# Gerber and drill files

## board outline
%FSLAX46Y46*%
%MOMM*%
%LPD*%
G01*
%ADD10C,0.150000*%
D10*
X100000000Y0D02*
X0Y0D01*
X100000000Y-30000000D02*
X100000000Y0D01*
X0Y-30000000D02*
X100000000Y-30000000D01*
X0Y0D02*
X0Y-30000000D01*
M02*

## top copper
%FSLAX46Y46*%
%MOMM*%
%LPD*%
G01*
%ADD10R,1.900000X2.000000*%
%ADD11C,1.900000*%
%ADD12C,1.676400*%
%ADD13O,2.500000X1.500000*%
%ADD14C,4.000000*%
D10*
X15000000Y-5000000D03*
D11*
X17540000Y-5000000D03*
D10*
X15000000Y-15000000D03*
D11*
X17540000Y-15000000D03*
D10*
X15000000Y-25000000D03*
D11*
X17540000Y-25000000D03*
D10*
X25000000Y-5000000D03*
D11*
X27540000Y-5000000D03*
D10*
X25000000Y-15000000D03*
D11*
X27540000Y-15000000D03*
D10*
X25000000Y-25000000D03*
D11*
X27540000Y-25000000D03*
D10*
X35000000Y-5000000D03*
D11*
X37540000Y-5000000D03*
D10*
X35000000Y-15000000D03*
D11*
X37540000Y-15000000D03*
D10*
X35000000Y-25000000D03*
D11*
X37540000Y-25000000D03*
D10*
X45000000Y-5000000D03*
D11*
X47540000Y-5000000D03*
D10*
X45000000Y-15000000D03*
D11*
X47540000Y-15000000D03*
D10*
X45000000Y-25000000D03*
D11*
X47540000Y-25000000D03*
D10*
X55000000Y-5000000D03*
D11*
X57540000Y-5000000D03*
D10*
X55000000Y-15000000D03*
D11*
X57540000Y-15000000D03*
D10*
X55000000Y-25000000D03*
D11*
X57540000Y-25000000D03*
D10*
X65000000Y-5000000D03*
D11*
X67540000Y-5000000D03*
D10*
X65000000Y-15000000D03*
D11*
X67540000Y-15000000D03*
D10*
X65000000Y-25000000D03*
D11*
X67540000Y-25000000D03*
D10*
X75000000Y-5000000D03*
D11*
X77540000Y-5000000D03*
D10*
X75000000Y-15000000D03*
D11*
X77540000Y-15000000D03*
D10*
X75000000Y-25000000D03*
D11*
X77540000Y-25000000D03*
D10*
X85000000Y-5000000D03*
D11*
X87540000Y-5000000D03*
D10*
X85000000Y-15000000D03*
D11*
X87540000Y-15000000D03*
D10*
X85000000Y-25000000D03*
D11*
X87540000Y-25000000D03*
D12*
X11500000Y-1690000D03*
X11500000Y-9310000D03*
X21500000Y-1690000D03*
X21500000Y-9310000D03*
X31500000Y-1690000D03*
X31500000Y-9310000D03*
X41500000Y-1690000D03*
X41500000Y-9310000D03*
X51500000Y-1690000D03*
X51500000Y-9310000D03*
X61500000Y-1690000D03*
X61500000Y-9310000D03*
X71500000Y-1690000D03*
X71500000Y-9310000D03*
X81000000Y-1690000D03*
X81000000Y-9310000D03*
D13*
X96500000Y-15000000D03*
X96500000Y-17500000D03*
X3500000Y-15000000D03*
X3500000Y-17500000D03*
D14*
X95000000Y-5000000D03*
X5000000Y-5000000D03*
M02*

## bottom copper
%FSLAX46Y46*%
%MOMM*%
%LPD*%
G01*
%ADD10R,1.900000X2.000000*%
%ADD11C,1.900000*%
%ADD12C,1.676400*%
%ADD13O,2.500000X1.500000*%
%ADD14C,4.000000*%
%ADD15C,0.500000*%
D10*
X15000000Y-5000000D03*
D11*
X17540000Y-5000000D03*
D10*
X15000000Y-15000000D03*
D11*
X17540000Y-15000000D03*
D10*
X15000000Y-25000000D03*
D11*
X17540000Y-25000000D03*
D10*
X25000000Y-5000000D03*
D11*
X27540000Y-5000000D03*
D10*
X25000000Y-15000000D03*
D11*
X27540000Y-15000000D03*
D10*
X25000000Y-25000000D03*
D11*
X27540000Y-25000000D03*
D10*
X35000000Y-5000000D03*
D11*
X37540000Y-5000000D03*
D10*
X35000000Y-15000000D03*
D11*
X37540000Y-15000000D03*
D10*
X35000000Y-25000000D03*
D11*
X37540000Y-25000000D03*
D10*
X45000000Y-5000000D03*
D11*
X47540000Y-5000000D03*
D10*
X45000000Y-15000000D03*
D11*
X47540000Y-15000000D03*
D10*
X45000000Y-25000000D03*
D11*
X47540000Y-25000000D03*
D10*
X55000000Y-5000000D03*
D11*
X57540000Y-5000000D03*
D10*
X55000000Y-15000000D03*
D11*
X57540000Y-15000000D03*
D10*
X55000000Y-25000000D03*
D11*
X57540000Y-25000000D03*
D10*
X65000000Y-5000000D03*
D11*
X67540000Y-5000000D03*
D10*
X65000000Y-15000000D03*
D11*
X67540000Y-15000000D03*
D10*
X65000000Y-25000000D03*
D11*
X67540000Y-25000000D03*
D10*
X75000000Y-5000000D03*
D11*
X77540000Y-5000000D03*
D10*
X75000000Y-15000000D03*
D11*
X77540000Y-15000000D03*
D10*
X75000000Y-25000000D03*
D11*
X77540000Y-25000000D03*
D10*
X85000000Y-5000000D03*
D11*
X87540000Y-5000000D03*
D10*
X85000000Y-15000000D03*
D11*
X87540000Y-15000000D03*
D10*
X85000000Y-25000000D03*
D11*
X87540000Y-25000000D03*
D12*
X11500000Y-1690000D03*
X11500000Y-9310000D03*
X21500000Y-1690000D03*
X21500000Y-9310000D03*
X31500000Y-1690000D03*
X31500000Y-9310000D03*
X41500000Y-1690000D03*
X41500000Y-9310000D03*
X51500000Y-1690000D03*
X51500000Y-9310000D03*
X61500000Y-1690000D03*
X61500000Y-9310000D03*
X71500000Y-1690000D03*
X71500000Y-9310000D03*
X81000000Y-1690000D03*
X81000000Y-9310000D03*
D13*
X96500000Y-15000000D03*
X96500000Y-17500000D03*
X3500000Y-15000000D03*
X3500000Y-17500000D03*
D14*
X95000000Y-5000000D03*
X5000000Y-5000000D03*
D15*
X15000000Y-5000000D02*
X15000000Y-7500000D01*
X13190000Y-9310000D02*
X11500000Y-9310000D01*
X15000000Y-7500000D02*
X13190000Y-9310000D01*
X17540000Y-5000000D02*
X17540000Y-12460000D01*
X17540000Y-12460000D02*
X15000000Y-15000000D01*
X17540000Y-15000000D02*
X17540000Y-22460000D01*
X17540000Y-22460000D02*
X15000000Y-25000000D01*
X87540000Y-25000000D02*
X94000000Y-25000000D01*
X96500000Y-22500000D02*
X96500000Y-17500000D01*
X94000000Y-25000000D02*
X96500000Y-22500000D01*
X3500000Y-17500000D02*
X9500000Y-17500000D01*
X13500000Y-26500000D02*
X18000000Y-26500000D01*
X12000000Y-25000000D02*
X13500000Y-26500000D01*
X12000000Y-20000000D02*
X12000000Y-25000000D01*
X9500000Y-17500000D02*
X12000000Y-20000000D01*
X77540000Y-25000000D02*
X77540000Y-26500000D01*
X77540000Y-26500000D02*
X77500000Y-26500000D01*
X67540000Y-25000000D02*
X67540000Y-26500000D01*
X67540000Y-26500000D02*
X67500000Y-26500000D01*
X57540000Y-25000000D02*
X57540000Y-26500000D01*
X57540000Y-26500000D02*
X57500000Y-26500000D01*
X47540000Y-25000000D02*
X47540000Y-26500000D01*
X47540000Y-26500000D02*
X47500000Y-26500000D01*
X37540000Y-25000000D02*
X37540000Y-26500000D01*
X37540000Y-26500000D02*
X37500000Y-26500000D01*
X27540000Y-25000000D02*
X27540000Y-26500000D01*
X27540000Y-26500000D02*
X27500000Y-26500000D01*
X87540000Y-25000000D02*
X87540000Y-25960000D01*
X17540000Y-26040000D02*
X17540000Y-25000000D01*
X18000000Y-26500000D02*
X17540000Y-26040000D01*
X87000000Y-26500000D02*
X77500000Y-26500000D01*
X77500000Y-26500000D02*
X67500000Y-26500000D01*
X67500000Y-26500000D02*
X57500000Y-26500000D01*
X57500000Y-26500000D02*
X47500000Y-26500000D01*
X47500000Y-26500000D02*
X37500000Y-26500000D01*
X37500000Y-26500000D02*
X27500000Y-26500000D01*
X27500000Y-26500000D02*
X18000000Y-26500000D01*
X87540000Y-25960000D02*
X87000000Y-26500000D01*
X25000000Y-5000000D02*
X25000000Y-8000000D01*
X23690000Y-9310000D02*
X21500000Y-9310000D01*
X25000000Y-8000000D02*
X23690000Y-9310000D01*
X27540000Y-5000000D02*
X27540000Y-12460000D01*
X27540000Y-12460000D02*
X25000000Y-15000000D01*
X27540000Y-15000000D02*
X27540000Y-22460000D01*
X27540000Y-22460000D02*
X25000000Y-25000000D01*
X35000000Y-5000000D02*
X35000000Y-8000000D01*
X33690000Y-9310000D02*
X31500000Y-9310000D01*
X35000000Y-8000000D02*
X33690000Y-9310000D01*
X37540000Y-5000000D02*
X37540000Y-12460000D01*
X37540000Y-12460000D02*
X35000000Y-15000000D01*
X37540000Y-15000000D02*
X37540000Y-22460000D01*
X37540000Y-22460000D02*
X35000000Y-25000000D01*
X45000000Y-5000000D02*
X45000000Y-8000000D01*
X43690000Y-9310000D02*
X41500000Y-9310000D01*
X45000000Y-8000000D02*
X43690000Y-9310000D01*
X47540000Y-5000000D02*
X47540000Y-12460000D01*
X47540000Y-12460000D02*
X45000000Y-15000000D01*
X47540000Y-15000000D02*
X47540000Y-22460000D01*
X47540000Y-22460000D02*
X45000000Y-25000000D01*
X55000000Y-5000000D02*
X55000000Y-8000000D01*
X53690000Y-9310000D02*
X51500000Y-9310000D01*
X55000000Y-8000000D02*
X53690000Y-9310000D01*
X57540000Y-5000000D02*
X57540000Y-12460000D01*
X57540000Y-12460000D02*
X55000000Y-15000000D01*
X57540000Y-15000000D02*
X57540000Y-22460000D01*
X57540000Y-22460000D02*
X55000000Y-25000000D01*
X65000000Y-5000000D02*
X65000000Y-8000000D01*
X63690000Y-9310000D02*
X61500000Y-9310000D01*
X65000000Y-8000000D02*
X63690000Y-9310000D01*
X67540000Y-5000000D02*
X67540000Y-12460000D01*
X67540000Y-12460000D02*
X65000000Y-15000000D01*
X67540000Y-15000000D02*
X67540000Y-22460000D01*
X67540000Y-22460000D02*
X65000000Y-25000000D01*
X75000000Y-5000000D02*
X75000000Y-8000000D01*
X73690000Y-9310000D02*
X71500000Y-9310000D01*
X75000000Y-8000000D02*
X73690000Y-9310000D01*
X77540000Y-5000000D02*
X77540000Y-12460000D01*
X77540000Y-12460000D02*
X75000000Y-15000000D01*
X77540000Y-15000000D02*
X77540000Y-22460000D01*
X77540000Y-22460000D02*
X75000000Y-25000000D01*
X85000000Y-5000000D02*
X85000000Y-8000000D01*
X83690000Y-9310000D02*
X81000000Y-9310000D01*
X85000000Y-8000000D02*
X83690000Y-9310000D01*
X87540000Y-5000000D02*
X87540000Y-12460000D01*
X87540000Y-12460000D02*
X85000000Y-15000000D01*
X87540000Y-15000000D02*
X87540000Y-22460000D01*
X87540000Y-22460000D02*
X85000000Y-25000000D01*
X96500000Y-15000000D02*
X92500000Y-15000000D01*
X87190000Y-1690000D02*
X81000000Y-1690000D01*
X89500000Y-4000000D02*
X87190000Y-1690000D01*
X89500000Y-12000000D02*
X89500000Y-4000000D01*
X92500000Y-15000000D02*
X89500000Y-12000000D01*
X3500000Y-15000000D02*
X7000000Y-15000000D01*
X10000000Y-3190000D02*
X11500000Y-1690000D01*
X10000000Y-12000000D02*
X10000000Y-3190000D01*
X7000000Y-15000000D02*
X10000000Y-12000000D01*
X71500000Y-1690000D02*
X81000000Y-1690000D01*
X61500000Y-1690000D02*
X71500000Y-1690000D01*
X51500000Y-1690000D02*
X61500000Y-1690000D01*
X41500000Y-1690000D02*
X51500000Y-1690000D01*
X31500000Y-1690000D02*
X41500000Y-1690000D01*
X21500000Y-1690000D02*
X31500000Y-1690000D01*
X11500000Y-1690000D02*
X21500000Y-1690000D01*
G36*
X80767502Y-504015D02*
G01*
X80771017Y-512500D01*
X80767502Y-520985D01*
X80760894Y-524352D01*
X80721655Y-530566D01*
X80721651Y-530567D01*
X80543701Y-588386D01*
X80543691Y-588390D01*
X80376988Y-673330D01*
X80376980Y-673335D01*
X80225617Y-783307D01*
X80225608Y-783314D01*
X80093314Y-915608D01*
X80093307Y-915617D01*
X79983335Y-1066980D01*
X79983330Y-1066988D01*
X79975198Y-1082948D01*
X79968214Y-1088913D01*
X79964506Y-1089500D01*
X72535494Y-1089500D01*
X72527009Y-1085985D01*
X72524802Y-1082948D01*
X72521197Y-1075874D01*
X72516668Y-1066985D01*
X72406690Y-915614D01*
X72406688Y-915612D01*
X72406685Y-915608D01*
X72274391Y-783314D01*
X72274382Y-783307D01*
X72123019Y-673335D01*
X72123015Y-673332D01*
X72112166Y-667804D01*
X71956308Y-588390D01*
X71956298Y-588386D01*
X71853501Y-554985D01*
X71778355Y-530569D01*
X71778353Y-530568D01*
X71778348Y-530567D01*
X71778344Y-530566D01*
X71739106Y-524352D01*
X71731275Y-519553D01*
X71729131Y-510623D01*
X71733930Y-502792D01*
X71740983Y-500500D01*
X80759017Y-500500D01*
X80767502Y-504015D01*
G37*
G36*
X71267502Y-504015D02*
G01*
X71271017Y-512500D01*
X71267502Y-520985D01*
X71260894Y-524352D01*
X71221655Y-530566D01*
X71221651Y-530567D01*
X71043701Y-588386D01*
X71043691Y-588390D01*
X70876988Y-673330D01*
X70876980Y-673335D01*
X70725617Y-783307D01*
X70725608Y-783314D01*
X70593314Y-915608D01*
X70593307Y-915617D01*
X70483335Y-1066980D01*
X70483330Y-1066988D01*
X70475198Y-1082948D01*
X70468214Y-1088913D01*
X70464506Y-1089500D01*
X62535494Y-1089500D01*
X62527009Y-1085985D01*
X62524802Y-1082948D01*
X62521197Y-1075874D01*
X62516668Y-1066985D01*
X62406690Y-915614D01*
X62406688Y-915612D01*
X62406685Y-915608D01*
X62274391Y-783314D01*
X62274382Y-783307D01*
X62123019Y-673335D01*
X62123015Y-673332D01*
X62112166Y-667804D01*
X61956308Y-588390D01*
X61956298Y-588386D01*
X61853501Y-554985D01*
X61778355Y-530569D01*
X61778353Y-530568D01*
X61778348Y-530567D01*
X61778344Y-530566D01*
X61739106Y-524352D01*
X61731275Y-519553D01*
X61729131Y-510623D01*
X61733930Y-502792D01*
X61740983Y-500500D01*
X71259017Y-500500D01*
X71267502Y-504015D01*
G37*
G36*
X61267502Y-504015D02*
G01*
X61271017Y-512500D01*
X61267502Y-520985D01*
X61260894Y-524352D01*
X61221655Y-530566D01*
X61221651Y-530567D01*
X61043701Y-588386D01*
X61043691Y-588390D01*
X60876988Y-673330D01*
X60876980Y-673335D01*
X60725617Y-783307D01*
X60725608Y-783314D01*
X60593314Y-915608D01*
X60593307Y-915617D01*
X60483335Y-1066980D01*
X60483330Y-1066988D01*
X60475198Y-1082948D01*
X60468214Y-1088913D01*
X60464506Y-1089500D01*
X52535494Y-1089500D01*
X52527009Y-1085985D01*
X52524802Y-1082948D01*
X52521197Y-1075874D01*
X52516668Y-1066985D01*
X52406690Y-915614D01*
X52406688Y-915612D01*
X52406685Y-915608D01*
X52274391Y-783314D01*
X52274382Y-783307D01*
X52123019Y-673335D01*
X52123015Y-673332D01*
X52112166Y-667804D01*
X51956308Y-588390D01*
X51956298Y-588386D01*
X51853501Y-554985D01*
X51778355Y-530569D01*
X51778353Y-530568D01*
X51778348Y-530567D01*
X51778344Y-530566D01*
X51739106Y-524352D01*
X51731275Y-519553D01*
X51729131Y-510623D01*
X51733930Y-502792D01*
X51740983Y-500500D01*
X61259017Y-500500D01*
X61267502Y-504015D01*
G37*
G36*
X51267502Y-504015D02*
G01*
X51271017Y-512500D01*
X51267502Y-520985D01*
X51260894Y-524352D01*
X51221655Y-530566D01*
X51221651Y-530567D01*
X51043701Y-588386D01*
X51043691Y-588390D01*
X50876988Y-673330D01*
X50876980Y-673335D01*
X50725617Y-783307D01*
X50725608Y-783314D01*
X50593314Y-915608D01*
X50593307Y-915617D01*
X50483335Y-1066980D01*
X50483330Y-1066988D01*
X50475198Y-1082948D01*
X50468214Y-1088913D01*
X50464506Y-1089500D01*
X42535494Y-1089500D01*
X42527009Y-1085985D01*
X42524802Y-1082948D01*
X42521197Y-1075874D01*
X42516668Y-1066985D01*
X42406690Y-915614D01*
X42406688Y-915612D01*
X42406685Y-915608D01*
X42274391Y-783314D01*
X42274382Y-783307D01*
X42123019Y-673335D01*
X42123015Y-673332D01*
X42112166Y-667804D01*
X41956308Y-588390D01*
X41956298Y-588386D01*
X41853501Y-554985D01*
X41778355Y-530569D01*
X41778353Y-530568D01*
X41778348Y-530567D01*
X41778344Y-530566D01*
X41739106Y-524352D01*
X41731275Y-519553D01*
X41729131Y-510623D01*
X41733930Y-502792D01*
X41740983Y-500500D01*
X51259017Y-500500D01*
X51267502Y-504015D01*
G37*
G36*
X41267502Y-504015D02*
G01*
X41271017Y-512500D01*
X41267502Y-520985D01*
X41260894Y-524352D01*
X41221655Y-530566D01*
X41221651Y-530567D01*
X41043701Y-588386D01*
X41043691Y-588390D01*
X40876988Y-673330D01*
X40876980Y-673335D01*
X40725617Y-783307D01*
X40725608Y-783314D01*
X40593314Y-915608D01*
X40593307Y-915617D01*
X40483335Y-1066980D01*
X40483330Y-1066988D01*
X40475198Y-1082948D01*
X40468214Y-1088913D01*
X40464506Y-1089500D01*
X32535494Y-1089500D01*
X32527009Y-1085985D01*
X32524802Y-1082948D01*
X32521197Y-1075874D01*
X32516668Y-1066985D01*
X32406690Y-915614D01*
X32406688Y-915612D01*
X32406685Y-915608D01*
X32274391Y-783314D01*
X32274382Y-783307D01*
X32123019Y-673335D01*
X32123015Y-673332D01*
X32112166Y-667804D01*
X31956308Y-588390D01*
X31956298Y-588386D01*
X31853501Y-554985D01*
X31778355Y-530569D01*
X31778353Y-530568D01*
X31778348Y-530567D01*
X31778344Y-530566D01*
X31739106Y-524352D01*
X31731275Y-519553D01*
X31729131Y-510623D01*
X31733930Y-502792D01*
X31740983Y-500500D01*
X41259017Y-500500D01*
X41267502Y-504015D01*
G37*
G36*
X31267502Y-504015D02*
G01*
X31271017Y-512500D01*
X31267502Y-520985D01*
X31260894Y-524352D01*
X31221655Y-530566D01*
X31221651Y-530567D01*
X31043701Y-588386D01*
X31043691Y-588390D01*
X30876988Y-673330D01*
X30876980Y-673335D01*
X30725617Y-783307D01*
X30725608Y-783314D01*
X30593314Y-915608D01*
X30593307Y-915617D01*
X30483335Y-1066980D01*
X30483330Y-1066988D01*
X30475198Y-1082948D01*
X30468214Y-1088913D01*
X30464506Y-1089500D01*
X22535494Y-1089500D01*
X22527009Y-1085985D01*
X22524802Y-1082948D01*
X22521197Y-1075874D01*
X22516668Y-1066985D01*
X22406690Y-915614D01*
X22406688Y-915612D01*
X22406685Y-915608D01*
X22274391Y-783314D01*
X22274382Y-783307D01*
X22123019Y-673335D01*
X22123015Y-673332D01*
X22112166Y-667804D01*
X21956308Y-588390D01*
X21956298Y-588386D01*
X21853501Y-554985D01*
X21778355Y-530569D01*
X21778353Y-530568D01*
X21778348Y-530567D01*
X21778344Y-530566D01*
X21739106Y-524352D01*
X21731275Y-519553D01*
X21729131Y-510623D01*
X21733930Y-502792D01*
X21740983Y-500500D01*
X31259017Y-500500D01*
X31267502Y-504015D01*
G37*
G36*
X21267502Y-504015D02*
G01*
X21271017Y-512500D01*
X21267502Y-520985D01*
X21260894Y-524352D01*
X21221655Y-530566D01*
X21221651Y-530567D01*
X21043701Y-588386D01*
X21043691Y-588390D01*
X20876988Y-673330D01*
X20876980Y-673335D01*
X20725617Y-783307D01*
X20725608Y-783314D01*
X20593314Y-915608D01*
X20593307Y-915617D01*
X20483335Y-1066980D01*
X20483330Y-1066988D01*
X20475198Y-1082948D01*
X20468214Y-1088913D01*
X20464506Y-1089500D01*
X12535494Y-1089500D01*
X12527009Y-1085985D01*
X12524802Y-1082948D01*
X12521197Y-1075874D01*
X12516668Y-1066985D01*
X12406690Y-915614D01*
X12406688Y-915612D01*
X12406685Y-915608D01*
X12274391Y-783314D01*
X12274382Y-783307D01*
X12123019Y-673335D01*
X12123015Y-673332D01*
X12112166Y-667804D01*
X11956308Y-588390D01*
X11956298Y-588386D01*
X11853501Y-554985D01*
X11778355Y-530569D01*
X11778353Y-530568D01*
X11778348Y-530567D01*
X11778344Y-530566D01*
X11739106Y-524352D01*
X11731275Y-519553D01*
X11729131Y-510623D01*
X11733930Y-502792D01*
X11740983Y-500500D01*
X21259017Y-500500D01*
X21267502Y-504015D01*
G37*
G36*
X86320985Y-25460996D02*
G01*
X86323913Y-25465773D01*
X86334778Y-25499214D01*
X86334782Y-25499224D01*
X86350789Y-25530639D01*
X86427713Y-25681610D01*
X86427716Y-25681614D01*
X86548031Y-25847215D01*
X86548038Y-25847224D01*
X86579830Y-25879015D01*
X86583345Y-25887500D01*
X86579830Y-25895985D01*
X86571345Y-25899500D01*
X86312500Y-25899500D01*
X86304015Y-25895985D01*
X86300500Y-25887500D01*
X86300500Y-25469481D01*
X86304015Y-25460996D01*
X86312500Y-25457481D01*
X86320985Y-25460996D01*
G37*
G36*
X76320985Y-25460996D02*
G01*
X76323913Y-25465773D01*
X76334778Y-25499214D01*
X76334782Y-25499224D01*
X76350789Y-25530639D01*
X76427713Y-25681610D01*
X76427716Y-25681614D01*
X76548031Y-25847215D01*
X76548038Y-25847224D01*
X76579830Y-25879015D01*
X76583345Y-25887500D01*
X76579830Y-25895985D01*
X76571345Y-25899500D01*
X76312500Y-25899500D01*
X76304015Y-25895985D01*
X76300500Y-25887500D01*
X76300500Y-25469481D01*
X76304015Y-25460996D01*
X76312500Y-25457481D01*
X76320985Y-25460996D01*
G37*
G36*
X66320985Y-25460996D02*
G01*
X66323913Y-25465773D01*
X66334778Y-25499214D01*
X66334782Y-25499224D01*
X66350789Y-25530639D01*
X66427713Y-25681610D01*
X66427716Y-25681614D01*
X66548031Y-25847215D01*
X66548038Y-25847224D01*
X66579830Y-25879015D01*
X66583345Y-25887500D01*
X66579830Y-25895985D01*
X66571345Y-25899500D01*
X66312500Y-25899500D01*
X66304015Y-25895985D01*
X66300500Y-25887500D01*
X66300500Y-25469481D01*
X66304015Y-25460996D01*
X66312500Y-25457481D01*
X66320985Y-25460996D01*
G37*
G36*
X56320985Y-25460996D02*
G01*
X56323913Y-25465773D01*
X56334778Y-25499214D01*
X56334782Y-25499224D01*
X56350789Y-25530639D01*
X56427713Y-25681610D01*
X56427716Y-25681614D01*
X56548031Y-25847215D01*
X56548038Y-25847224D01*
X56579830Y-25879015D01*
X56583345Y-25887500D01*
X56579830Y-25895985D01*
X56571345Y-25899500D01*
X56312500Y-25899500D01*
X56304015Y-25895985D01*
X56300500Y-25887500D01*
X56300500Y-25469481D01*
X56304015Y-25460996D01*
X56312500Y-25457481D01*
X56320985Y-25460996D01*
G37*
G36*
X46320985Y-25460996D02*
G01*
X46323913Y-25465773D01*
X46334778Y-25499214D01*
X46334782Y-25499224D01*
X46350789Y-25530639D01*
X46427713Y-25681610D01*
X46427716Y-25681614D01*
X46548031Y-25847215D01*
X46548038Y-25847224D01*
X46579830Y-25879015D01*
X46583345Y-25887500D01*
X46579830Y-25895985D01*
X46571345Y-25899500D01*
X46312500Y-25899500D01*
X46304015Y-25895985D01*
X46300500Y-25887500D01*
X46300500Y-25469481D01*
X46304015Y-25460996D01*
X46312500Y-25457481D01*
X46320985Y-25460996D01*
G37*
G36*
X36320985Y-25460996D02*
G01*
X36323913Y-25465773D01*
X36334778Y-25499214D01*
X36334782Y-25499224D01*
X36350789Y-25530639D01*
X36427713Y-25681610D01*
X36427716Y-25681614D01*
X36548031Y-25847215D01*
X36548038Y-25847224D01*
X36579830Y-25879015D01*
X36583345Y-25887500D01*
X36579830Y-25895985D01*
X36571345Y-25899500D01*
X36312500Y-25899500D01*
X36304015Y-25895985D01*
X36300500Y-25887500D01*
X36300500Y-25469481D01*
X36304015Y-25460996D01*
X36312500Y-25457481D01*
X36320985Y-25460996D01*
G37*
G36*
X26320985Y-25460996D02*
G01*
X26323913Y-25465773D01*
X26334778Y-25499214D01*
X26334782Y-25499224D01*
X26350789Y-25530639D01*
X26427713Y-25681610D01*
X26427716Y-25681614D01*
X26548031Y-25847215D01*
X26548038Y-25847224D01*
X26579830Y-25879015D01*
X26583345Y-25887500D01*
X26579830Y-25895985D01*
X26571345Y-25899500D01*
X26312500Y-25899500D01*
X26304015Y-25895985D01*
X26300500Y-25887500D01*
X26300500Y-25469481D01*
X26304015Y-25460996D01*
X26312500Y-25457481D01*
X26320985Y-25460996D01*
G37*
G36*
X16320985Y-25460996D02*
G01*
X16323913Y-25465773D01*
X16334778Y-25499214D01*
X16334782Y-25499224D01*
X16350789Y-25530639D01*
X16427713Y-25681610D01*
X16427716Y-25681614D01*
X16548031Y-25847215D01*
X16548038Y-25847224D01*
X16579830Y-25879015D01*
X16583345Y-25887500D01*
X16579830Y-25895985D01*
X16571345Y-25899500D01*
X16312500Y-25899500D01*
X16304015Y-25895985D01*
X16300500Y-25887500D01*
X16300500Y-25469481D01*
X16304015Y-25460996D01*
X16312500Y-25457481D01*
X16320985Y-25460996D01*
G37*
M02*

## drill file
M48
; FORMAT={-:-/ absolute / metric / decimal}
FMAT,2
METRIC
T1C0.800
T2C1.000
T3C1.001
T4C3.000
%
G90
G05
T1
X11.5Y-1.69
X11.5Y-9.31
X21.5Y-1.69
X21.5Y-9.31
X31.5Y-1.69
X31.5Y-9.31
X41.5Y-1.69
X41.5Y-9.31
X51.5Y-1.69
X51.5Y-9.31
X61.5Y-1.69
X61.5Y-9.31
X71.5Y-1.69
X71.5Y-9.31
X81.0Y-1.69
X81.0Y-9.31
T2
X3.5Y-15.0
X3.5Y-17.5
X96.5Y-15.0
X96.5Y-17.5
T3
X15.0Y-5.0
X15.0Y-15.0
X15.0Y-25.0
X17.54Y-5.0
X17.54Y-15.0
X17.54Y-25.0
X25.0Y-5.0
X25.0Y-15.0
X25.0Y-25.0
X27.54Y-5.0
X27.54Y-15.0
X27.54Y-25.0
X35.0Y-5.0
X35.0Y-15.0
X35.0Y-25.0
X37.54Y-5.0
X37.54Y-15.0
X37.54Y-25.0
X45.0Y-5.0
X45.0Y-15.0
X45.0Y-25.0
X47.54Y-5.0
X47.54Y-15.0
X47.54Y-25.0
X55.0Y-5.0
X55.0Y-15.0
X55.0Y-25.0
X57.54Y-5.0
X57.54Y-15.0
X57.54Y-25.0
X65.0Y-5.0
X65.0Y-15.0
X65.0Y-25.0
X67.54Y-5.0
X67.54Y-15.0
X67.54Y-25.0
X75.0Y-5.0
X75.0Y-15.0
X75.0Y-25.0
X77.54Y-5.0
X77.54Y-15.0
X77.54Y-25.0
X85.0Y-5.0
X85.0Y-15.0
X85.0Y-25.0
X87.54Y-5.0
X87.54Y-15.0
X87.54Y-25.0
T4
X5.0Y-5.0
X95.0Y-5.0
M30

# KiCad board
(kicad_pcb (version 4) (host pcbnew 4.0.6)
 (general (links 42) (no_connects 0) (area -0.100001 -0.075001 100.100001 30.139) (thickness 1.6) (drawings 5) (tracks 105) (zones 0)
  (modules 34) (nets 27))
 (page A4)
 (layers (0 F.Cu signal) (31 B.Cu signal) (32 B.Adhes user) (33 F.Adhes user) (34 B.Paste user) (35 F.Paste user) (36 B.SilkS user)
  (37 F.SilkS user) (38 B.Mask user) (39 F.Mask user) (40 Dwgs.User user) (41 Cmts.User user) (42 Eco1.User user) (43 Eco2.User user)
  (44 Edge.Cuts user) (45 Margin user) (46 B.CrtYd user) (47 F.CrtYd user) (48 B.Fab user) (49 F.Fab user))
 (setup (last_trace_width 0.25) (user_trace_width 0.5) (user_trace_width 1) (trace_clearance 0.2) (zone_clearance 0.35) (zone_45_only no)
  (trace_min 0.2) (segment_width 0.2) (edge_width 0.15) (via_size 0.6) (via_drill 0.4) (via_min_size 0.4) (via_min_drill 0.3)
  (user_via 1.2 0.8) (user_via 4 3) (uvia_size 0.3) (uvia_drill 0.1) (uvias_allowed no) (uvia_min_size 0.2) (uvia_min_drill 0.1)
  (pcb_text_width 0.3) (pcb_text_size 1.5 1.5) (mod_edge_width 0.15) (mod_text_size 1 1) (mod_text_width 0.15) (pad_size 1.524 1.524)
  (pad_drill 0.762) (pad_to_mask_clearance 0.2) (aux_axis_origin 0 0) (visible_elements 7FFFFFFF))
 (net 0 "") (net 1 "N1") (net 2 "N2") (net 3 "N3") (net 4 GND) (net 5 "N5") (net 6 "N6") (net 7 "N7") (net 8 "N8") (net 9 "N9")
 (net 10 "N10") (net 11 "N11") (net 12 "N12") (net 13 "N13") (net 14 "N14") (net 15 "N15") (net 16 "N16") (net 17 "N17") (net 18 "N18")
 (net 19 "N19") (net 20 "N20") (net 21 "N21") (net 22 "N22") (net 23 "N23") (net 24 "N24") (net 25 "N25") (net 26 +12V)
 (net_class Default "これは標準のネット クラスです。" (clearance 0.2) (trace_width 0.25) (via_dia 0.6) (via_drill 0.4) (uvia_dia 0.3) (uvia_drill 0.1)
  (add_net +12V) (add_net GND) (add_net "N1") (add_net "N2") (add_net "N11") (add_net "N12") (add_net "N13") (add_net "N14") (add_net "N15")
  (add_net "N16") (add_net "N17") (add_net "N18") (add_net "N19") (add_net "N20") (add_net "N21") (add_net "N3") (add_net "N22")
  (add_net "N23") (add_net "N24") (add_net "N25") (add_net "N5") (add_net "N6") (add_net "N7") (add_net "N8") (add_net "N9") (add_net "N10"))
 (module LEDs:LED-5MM (layer F.Cu) (at 15 5)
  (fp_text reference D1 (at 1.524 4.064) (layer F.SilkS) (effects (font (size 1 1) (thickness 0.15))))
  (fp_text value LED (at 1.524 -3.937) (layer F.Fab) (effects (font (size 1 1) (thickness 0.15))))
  (pad 1 thru_hole rect (at 0 0 90) (size 2 1.9) (drill 1.00076) (layers *.Cu *.Mask F.SilkS) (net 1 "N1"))
  (pad 2 thru_hole circle (at 2.54 0) (size 1.9 1.9) (drill 1.00076) (layers *.Cu *.Mask F.SilkS) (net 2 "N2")))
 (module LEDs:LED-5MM (layer F.Cu) (at 15 15)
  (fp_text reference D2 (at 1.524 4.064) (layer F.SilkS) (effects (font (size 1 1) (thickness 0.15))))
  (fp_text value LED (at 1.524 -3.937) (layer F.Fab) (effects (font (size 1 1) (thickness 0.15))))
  (pad 1 thru_hole rect (at 0 0 90) (size 2 1.9) (drill 1.00076) (layers *.Cu *.Mask F.SilkS) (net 2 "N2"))
  (pad 2 thru_hole circle (at 2.54 0) (size 1.9 1.9) (drill 1.00076) (layers *.Cu *.Mask F.SilkS) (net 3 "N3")))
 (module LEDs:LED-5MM (layer F.Cu) (at 15 25)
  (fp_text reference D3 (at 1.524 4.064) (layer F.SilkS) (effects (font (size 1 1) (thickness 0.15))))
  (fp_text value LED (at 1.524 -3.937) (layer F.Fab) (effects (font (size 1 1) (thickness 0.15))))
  (pad 1 thru_hole rect (at 0 0 90) (size 2 1.9) (drill 1.00076) (layers *.Cu *.Mask F.SilkS) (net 3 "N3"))
  (pad 2 thru_hole circle (at 2.54 0) (size 1.9 1.9) (drill 1.00076) (layers *.Cu *.Mask F.SilkS) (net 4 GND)))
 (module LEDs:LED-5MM (layer F.Cu) (at 25 5)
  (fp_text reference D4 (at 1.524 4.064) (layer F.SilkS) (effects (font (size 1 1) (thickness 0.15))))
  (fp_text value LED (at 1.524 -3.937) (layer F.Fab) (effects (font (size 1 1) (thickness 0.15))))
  (pad 1 thru_hole rect (at 0 0 90) (size 2 1.9) (drill 1.00076) (layers *.Cu *.Mask F.SilkS) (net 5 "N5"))
  (pad 2 thru_hole circle (at 2.54 0) (size 1.9 1.9) (drill 1.00076) (layers *.Cu *.Mask F.SilkS) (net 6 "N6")))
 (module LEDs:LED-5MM (layer F.Cu) (at 25 15)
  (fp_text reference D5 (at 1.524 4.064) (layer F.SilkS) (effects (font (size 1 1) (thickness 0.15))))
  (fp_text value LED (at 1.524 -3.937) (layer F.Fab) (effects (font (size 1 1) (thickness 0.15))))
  (pad 1 thru_hole rect (at 0 0 90) (size 2 1.9) (drill 1.00076) (layers *.Cu *.Mask F.SilkS) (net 6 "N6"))
  (pad 2 thru_hole circle (at 2.54 0) (size 1.9 1.9) (drill 1.00076) (layers *.Cu *.Mask F.SilkS) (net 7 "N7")))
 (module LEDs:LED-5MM (layer F.Cu) (at 25 25)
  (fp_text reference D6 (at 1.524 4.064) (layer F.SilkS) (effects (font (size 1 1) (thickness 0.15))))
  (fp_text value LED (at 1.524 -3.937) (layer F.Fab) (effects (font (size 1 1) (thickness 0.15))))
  (pad 1 thru_hole rect (at 0 0 90) (size 2 1.9) (drill 1.00076) (layers *.Cu *.Mask F.SilkS) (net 7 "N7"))
  (pad 2 thru_hole circle (at 2.54 0) (size 1.9 1.9) (drill 1.00076) (layers *.Cu *.Mask F.SilkS) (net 4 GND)))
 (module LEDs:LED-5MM (layer F.Cu) (at 35 5)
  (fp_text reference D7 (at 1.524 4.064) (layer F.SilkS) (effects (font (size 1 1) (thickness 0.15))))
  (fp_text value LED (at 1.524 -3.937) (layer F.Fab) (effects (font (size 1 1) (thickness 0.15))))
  (pad 1 thru_hole rect (at 0 0 90) (size 2 1.9) (drill 1.00076) (layers *.Cu *.Mask F.SilkS) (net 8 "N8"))
  (pad 2 thru_hole circle (at 2.54 0) (size 1.9 1.9) (drill 1.00076) (layers *.Cu *.Mask F.SilkS) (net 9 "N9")))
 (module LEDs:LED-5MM (layer F.Cu) (at 35 15)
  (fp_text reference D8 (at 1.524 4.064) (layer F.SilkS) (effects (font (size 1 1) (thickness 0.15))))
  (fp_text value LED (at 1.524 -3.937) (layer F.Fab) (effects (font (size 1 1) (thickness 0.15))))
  (pad 1 thru_hole rect (at 0 0 90) (size 2 1.9) (drill 1.00076) (layers *.Cu *.Mask F.SilkS) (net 9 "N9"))
  (pad 2 thru_hole circle (at 2.54 0) (size 1.9 1.9) (drill 1.00076) (layers *.Cu *.Mask F.SilkS) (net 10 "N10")))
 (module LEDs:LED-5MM (layer F.Cu) (at 35 25)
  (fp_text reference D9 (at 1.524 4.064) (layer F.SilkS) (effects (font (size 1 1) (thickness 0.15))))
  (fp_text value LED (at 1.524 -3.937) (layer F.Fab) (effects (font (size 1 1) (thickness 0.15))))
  (pad 1 thru_hole rect (at 0 0 90) (size 2 1.9) (drill 1.00076) (layers *.Cu *.Mask F.SilkS) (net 10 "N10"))
  (pad 2 thru_hole circle (at 2.54 0) (size 1.9 1.9) (drill 1.00076) (layers *.Cu *.Mask F.SilkS) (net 4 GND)))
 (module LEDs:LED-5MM (layer F.Cu) (at 45 5)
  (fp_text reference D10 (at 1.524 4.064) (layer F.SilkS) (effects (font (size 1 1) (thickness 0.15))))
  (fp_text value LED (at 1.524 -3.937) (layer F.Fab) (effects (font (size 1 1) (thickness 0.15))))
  (pad 1 thru_hole rect (at 0 0 90) (size 2 1.9) (drill 1.00076) (layers *.Cu *.Mask F.SilkS) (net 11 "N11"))
  (pad 2 thru_hole circle (at 2.54 0) (size 1.9 1.9) (drill 1.00076) (layers *.Cu *.Mask F.SilkS) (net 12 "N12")))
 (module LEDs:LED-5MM (layer F.Cu) (at 45 15)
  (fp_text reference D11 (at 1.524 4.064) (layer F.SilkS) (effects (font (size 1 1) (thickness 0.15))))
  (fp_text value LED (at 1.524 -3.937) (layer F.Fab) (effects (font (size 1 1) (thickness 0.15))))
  (pad 1 thru_hole rect (at 0 0 90) (size 2 1.9) (drill 1.00076) (layers *.Cu *.Mask F.SilkS) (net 12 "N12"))
  (pad 2 thru_hole circle (at 2.54 0) (size 1.9 1.9) (drill 1.00076) (layers *.Cu *.Mask F.SilkS) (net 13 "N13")))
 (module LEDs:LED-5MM (layer F.Cu) (at 45 25)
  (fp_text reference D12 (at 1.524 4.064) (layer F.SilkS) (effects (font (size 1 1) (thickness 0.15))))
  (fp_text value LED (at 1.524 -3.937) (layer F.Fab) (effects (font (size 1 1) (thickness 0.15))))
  (pad 1 thru_hole rect (at 0 0 90) (size 2 1.9) (drill 1.00076) (layers *.Cu *.Mask F.SilkS) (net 13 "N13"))
  (pad 2 thru_hole circle (at 2.54 0) (size 1.9 1.9) (drill 1.00076) (layers *.Cu *.Mask F.SilkS) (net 4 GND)))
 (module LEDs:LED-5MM (layer F.Cu) (at 55 5)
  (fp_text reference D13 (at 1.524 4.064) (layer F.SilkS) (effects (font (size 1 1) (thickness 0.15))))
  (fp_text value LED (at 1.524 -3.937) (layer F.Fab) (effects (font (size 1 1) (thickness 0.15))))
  (pad 1 thru_hole rect (at 0 0 90) (size 2 1.9) (drill 1.00076) (layers *.Cu *.Mask F.SilkS) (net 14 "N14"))
  (pad 2 thru_hole circle (at 2.54 0) (size 1.9 1.9) (drill 1.00076) (layers *.Cu *.Mask F.SilkS) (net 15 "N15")))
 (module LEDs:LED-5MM (layer F.Cu) (at 55 15)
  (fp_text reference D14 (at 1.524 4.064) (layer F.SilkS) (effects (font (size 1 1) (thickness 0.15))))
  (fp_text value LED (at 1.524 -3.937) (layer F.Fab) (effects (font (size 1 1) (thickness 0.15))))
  (pad 1 thru_hole rect (at 0 0 90) (size 2 1.9) (drill 1.00076) (layers *.Cu *.Mask F.SilkS) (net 15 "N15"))
  (pad 2 thru_hole circle (at 2.54 0) (size 1.9 1.9) (drill 1.00076) (layers *.Cu *.Mask F.SilkS) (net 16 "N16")))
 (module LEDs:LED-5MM (layer F.Cu) (at 55 25)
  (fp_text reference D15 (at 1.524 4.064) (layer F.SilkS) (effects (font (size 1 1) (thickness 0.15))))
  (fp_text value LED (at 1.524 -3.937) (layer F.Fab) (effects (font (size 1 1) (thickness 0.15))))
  (pad 1 thru_hole rect (at 0 0 90) (size 2 1.9) (drill 1.00076) (layers *.Cu *.Mask F.SilkS) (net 16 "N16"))
  (pad 2 thru_hole circle (at 2.54 0) (size 1.9 1.9) (drill 1.00076) (layers *.Cu *.Mask F.SilkS) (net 4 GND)))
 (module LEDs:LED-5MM (layer F.Cu) (at 65 5)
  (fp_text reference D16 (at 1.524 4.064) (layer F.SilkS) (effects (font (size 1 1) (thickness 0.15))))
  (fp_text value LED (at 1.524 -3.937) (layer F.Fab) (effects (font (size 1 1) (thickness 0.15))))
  (pad 1 thru_hole rect (at 0 0 90) (size 2 1.9) (drill 1.00076) (layers *.Cu *.Mask F.SilkS) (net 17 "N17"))
  (pad 2 thru_hole circle (at 2.54 0) (size 1.9 1.9) (drill 1.00076) (layers *.Cu *.Mask F.SilkS) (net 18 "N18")))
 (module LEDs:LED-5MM (layer F.Cu) (at 65 15)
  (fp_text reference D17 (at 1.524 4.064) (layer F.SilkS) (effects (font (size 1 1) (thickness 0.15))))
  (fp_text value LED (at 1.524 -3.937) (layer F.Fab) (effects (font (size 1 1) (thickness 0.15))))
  (pad 1 thru_hole rect (at 0 0 90) (size 2 1.9) (drill 1.00076) (layers *.Cu *.Mask F.SilkS) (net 18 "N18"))
  (pad 2 thru_hole circle (at 2.54 0) (size 1.9 1.9) (drill 1.00076) (layers *.Cu *.Mask F.SilkS) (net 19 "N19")))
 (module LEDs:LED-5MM (layer F.Cu) (at 65 25)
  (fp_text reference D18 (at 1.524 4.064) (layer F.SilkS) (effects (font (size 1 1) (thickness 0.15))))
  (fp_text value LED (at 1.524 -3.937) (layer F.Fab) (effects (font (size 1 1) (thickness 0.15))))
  (pad 1 thru_hole rect (at 0 0 90) (size 2 1.9) (drill 1.00076) (layers *.Cu *.Mask F.SilkS) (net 19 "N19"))
  (pad 2 thru_hole circle (at 2.54 0) (size 1.9 1.9) (drill 1.00076) (layers *.Cu *.Mask F.SilkS) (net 4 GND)))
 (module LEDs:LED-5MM (layer F.Cu) (at 75 5)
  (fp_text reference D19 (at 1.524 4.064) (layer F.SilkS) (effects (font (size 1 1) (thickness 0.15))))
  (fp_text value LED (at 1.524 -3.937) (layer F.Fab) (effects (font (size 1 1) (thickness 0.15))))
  (pad 1 thru_hole rect (at 0 0 90) (size 2 1.9) (drill 1.00076) (layers *.Cu *.Mask F.SilkS) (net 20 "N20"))
  (pad 2 thru_hole circle (at 2.54 0) (size 1.9 1.9) (drill 1.00076) (layers *.Cu *.Mask F.SilkS) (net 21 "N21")))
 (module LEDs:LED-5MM (layer F.Cu) (at 75 15)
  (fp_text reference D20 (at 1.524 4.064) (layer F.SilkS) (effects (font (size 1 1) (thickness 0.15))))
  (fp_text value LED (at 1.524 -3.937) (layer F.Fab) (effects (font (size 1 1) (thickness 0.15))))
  (pad 1 thru_hole rect (at 0 0 90) (size 2 1.9) (drill 1.00076) (layers *.Cu *.Mask F.SilkS) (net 21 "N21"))
  (pad 2 thru_hole circle (at 2.54 0) (size 1.9 1.9) (drill 1.00076) (layers *.Cu *.Mask F.SilkS) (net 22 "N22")))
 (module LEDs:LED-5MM (layer F.Cu) (at 75 25)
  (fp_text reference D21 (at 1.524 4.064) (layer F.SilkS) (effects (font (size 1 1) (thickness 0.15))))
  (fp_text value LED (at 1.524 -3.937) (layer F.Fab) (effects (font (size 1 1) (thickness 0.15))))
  (pad 1 thru_hole rect (at 0 0 90) (size 2 1.9) (drill 1.00076) (layers *.Cu *.Mask F.SilkS) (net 22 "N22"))
  (pad 2 thru_hole circle (at 2.54 0) (size 1.9 1.9) (drill 1.00076) (layers *.Cu *.Mask F.SilkS) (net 4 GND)))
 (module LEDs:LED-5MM (layer F.Cu) (at 85 5)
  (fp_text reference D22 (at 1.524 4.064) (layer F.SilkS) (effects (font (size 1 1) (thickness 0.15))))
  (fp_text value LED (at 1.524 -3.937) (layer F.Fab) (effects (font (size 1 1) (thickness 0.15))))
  (pad 1 thru_hole rect (at 0 0 90) (size 2 1.9) (drill 1.00076) (layers *.Cu *.Mask F.SilkS) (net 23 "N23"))
  (pad 2 thru_hole circle (at 2.54 0) (size 1.9 1.9) (drill 1.00076) (layers *.Cu *.Mask F.SilkS) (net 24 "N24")))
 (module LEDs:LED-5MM (layer F.Cu) (at 85 15)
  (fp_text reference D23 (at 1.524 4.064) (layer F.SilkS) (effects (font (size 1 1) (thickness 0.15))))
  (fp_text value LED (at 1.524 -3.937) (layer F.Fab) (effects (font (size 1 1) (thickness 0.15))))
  (pad 1 thru_hole rect (at 0 0 90) (size 2 1.9) (drill 1.00076) (layers *.Cu *.Mask F.SilkS) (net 24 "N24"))
  (pad 2 thru_hole circle (at 2.54 0) (size 1.9 1.9) (drill 1.00076) (layers *.Cu *.Mask F.SilkS) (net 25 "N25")))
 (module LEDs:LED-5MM (layer F.Cu) (at 85 25)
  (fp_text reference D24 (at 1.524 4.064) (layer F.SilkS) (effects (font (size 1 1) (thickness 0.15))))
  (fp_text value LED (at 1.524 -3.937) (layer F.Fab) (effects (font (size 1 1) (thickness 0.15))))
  (pad 1 thru_hole rect (at 0 0 90) (size 2 1.9) (drill 1.00076) (layers *.Cu *.Mask F.SilkS) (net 25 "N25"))
  (pad 2 thru_hole circle (at 2.54 0) (size 1.9 1.9) (drill 1.00076) (layers *.Cu *.Mask F.SilkS) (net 4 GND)))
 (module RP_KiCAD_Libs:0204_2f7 (layer F.Cu) (at 11.5 5.5 270)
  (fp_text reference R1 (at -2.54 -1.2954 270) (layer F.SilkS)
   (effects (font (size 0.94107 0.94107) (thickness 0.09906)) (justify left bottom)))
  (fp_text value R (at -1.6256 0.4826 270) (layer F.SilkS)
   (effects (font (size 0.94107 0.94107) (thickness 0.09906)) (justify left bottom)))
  (pad 1 thru_hole circle (at -3.81 0 270) (size 1.6764 1.6764) (drill 0.8) (layers *.Cu *.Mask) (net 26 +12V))
  (pad 2 thru_hole circle (at 3.81 0 270) (size 1.6764 1.6764) (drill 0.8) (layers *.Cu *.Mask) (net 1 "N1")))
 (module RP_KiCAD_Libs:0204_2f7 (layer F.Cu) (at 21.5 5.5 270)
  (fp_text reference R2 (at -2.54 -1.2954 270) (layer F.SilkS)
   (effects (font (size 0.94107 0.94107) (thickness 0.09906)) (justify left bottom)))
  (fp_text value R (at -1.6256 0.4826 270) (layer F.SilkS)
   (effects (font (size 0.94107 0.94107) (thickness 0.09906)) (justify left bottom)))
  (pad 1 thru_hole circle (at -3.81 0 270) (size 1.6764 1.6764) (drill 0.8) (layers *.Cu *.Mask) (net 26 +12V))
  (pad 2 thru_hole circle (at 3.81 0 270) (size 1.6764 1.6764) (drill 0.8) (layers *.Cu *.Mask) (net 5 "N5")))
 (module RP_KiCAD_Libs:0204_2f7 (layer F.Cu) (at 31.5 5.5 270)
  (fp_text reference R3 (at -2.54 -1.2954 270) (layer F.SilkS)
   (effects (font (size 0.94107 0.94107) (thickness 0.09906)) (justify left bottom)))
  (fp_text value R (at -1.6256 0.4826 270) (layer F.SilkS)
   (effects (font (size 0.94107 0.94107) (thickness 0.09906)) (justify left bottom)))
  (pad 1 thru_hole circle (at -3.81 0 270) (size 1.6764 1.6764) (drill 0.8) (layers *.Cu *.Mask) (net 26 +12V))
  (pad 2 thru_hole circle (at 3.81 0 270) (size 1.6764 1.6764) (drill 0.8) (layers *.Cu *.Mask) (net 8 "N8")))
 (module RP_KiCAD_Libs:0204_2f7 (layer F.Cu) (at 41.5 5.5 270)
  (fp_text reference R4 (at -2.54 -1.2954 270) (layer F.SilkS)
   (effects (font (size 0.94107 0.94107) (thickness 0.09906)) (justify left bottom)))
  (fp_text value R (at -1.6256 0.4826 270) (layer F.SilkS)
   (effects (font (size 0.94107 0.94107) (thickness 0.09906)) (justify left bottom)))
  (pad 1 thru_hole circle (at -3.81 0 270) (size 1.6764 1.6764) (drill 0.8) (layers *.Cu *.Mask) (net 26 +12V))
  (pad 2 thru_hole circle (at 3.81 0 270) (size 1.6764 1.6764) (drill 0.8) (layers *.Cu *.Mask) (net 11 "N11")))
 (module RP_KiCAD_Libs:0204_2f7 (layer F.Cu) (at 51.5 5.5 270)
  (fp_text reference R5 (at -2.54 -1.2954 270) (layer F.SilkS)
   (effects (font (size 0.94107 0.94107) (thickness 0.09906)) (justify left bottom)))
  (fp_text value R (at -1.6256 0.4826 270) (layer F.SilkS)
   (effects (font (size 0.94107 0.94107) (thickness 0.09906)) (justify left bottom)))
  (pad 1 thru_hole circle (at -3.81 0 270) (size 1.6764 1.6764) (drill 0.8) (layers *.Cu *.Mask) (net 26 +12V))
  (pad 2 thru_hole circle (at 3.81 0 270) (size 1.6764 1.6764) (drill 0.8) (layers *.Cu *.Mask) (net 14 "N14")))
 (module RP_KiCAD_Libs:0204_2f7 (layer F.Cu) (at 61.5 5.5 270)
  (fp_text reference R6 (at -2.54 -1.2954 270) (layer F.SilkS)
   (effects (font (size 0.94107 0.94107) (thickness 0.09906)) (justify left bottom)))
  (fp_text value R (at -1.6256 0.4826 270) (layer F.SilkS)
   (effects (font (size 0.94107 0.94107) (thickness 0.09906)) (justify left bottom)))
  (pad 1 thru_hole circle (at -3.81 0 270) (size 1.6764 1.6764) (drill 0.8) (layers *.Cu *.Mask) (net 26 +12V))
  (pad 2 thru_hole circle (at 3.81 0 270) (size 1.6764 1.6764) (drill 0.8) (layers *.Cu *.Mask) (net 17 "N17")))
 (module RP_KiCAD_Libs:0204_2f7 (layer F.Cu) (at 71.5 5.5 270)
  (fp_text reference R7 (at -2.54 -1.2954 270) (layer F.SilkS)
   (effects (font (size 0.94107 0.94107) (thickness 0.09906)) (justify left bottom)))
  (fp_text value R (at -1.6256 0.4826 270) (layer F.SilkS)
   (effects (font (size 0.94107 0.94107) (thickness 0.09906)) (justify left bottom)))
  (pad 1 thru_hole circle (at -3.81 0 270) (size 1.6764 1.6764) (drill 0.8) (layers *.Cu *.Mask) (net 26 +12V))
  (pad 2 thru_hole circle (at 3.81 0 270) (size 1.6764 1.6764) (drill 0.8) (layers *.Cu *.Mask) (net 20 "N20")))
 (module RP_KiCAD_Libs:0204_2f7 (layer F.Cu) (at 81 5.5 270)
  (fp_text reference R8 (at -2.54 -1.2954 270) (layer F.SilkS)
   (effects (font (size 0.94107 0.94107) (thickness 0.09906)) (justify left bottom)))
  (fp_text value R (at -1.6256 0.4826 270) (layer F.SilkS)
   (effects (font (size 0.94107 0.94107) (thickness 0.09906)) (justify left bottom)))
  (pad 1 thru_hole circle (at -3.81 0 270) (size 1.6764 1.6764) (drill 0.8) (layers *.Cu *.Mask) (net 26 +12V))
  (pad 2 thru_hole circle (at 3.81 0 270) (size 1.6764 1.6764) (drill 0.8) (layers *.Cu *.Mask) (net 23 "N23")))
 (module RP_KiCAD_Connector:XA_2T (layer F.Cu) (at 96.5 15 270)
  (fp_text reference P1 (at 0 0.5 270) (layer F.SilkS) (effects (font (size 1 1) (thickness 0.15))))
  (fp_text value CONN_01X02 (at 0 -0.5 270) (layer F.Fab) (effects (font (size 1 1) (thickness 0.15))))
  (pad 2 thru_hole oval (at 0 0 270) (size 1.5 2.5) (drill 1) (layers *.Cu *.Mask F.SilkS) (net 26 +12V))
  (pad 1 thru_hole oval (at 2.5 0 270) (size 1.5 2.5) (drill 1) (layers *.Cu *.Mask F.SilkS) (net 4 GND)))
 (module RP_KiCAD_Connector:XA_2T (layer F.Cu) (at 3.5 15 270)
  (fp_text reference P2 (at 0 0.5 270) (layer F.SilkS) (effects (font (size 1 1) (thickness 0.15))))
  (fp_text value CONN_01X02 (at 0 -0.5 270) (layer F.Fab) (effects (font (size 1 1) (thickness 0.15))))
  (pad 2 thru_hole oval (at 0 0 270) (size 1.5 2.5) (drill 1) (layers *.Cu *.Mask F.SilkS) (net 26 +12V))
  (pad 1 thru_hole oval (at 2.5 0 270) (size 1.5 2.5) (drill 1) (layers *.Cu *.Mask F.SilkS) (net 4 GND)))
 (gr_line (start 100 0) (end 0 0) (angle 90) (layer Edge.Cuts) (width 0.15))
 (gr_line (start 100 30) (end 100 0) (angle 90) (layer Edge.Cuts) (width 0.15))
 (gr_line (start 0 30) (end 100 30) (angle 90) (layer Edge.Cuts) (width 0.15))
 (gr_line (start 0 0) (end 0 30) (angle 90) (layer Edge.Cuts) (width 0.15))
 (via (at 95 5) (size 4) (drill 3) (layers F.Cu B.Cu) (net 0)) (via (at 5 5) (size 4) (drill 3) (layers F.Cu B.Cu) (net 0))
 (segment (start 15 5) (end 15 7.5) (width 0.5) (layer B.Cu) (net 1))
 (segment (start 13.19 9.31) (end 11.5 9.31) (width 0.5) (layer B.Cu) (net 1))
 (segment (start 15 7.5) (end 13.19 9.31) (width 0.5) (layer B.Cu) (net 1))
 (segment (start 17.54 5) (end 17.54 12.46) (width 0.5) (layer B.Cu) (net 2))
 (segment (start 17.54 12.46) (end 15 15) (width 0.5) (layer B.Cu) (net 2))
 (segment (start 17.54 15) (end 17.54 22.46) (width 0.5) (layer B.Cu) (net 3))
 (segment (start 17.54 22.46) (end 15 25) (width 0.5) (layer B.Cu) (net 3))
 (segment (start 87.54 25) (end 94 25) (width 0.5) (layer B.Cu) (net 4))
 (segment (start 96.5 22.5) (end 96.5 17.5) (width 0.5) (layer B.Cu) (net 4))
 (segment (start 94 25) (end 96.5 22.5) (width 0.5) (layer B.Cu) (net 4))
 (segment (start 3.5 17.5) (end 9.5 17.5) (width 0.5) (layer B.Cu) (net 4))
 (segment (start 13.5 26.5) (end 18 26.5) (width 0.5) (layer B.Cu) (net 4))
 (segment (start 12 25) (end 13.5 26.5) (width 0.5) (layer B.Cu) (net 4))
 (segment (start 12 20) (end 12 25) (width 0.5) (layer B.Cu) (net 4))
 (segment (start 9.5 17.5) (end 12 20) (width 0.5) (layer B.Cu) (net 4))
 (segment (start 77.54 25) (end 77.54 26.5) (width 0.5) (layer B.Cu) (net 4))
 (segment (start 77.54 26.5) (end 77.5 26.5) (width 0.5) (layer B.Cu) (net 4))
 (segment (start 67.54 25) (end 67.54 26.5) (width 0.5) (layer B.Cu) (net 4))
 (segment (start 67.54 26.5) (end 67.5 26.5) (width 0.5) (layer B.Cu) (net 4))
 (segment (start 57.54 25) (end 57.54 26.5) (width 0.5) (layer B.Cu) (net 4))
 (segment (start 57.54 26.5) (end 57.5 26.5) (width 0.5) (layer B.Cu) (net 4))
 (segment (start 47.54 25) (end 47.54 26.5) (width 0.5) (layer B.Cu) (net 4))
 (segment (start 47.54 26.5) (end 47.5 26.5) (width 0.5) (layer B.Cu) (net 4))
 (segment (start 37.54 25) (end 37.54 26.5) (width 0.5) (layer B.Cu) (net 4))
 (segment (start 37.54 26.5) (end 37.5 26.5) (width 0.5) (layer B.Cu) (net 4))
 (segment (start 27.54 25) (end 27.54 26.5) (width 0.5) (layer B.Cu) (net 4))
 (segment (start 27.54 26.5) (end 27.5 26.5) (width 0.5) (layer B.Cu) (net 4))
 (segment (start 87.54 25) (end 87.54 25.96) (width 0.5) (layer B.Cu) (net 4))
 (segment (start 17.54 26.04) (end 17.54 25) (width 0.5) (layer B.Cu) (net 4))
 (segment (start 18 26.5) (end 17.54 26.04) (width 0.5) (layer B.Cu) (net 4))
 (segment (start 87 26.5) (end 77.5 26.5) (width 0.5) (layer B.Cu) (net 4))
 (segment (start 77.5 26.5) (end 67.5 26.5) (width 0.5) (layer B.Cu) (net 4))
 (segment (start 67.5 26.5) (end 57.5 26.5) (width 0.5) (layer B.Cu) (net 4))
 (segment (start 57.5 26.5) (end 47.5 26.5) (width 0.5) (layer B.Cu) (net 4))
 (segment (start 47.5 26.5) (end 37.5 26.5) (width 0.5) (layer B.Cu) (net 4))
 (segment (start 37.5 26.5) (end 27.5 26.5) (width 0.5) (layer B.Cu) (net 4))
 (segment (start 27.5 26.5) (end 18 26.5) (width 0.5) (layer B.Cu) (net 4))
 (segment (start 87.54 25.96) (end 87 26.5) (width 0.5) (layer B.Cu) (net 4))
 (segment (start 25 5) (end 25 8) (width 0.5) (layer B.Cu) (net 5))
 (segment (start 23.69 9.31) (end 21.5 9.31) (width 0.5) (layer B.Cu) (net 5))
 (segment (start 25 8) (end 23.69 9.31) (width 0.5) (layer B.Cu) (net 5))
 (segment (start 27.54 5) (end 27.54 12.46) (width 0.5) (layer B.Cu) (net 6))
 (segment (start 27.54 12.46) (end 25 15) (width 0.5) (layer B.Cu) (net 6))
 (segment (start 27.54 15) (end 27.54 22.46) (width 0.5) (layer B.Cu) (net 7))
 (segment (start 27.54 22.46) (end 25 25) (width 0.5) (layer B.Cu) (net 7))
 (segment (start 35 5) (end 35 8) (width 0.5) (layer B.Cu) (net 8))
 (segment (start 33.69 9.31) (end 31.5 9.31) (width 0.5) (layer B.Cu) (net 8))
 (segment (start 35 8) (end 33.69 9.31) (width 0.5) (layer B.Cu) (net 8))
 (segment (start 37.54 5) (end 37.54 12.46) (width 0.5) (layer B.Cu) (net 9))
 (segment (start 37.54 12.46) (end 35 15) (width 0.5) (layer B.Cu) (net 9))
 (segment (start 37.54 15) (end 37.54 22.46) (width 0.5) (layer B.Cu) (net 10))
 (segment (start 37.54 22.46) (end 35 25) (width 0.5) (layer B.Cu) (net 10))
 (segment (start 45 5) (end 45 8) (width 0.5) (layer B.Cu) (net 11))
 (segment (start 43.69 9.31) (end 41.5 9.31) (width 0.5) (layer B.Cu) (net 11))
 (segment (start 45 8) (end 43.69 9.31) (width 0.5) (layer B.Cu) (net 11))
 (segment (start 47.54 5) (end 47.54 12.46) (width 0.5) (layer B.Cu) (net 12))
 (segment (start 47.54 12.46) (end 45 15) (width 0.5) (layer B.Cu) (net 12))
 (segment (start 47.54 15) (end 47.54 22.46) (width 0.5) (layer B.Cu) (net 13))
 (segment (start 47.54 22.46) (end 45 25) (width 0.5) (layer B.Cu) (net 13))
 (segment (start 55 5) (end 55 8) (width 0.5) (layer B.Cu) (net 14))
 (segment (start 53.69 9.31) (end 51.5 9.31) (width 0.5) (layer B.Cu) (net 14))
 (segment (start 55 8) (end 53.69 9.31) (width 0.5) (layer B.Cu) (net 14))
 (segment (start 57.54 5) (end 57.54 12.46) (width 0.5) (layer B.Cu) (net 15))
 (segment (start 57.54 12.46) (end 55 15) (width 0.5) (layer B.Cu) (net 15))
 (segment (start 57.54 15) (end 57.54 22.46) (width 0.5) (layer B.Cu) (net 16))
 (segment (start 57.54 22.46) (end 55 25) (width 0.5) (layer B.Cu) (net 16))
 (segment (start 65 5) (end 65 8) (width 0.5) (layer B.Cu) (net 17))
 (segment (start 63.69 9.31) (end 61.5 9.31) (width 0.5) (layer B.Cu) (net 17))
 (segment (start 65 8) (end 63.69 9.31) (width 0.5) (layer B.Cu) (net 17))
 (segment (start 67.54 5) (end 67.54 12.46) (width 0.5) (layer B.Cu) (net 18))
 (segment (start 67.54 12.46) (end 65 15) (width 0.5) (layer B.Cu) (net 18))
 (segment (start 67.54 15) (end 67.54 22.46) (width 0.5) (layer B.Cu) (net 19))
 (segment (start 67.54 22.46) (end 65 25) (width 0.5) (layer B.Cu) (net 19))
 (segment (start 75 5) (end 75 8) (width 0.5) (layer B.Cu) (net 20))
 (segment (start 73.69 9.31) (end 71.5 9.31) (width 0.5) (layer B.Cu) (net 20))
 (segment (start 75 8) (end 73.69 9.31) (width 0.5) (layer B.Cu) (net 20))
 (segment (start 77.54 5) (end 77.54 12.46) (width 0.5) (layer B.Cu) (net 21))
 (segment (start 77.54 12.46) (end 75 15) (width 0.5) (layer B.Cu) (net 21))
 (segment (start 77.54 15) (end 77.54 22.46) (width 0.5) (layer B.Cu) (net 22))
 (segment (start 77.54 22.46) (end 75 25) (width 0.5) (layer B.Cu) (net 22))
 (segment (start 85 5) (end 85 8) (width 0.5) (layer B.Cu) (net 23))
 (segment (start 83.69 9.31) (end 81 9.31) (width 0.5) (layer B.Cu) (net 23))
 (segment (start 85 8) (end 83.69 9.31) (width 0.5) (layer B.Cu) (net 23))
 (segment (start 87.54 5) (end 87.54 12.46) (width 0.5) (layer B.Cu) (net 24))
 (segment (start 87.54 12.46) (end 85 15) (width 0.5) (layer B.Cu) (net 24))
 (segment (start 87.54 15) (end 87.54 22.46) (width 0.5) (layer B.Cu) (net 25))
 (segment (start 87.54 22.46) (end 85 25) (width 0.5) (layer B.Cu) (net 25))
 (segment (start 96.5 15) (end 92.5 15) (width 0.5) (layer B.Cu) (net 26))
 (segment (start 87.19 1.69) (end 81 1.69) (width 0.5) (layer B.Cu) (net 26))
 (segment (start 89.5 4) (end 87.19 1.69) (width 0.5) (layer B.Cu) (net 26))
 (segment (start 89.5 12) (end 89.5 4) (width 0.5) (layer B.Cu) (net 26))
 (segment (start 92.5 15) (end 89.5 12) (width 0.5) (layer B.Cu) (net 26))
 (segment (start 3.5 15) (end 7 15) (width 0.5) (layer B.Cu) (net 26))
 (segment (start 10 3.19) (end 11.5 1.69) (width 0.5) (layer B.Cu) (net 26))
 (segment (start 10 12) (end 10 3.19) (width 0.5) (layer B.Cu) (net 26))
 (segment (start 7 15) (end 10 12) (width 0.5) (layer B.Cu) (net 26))
 (segment (start 71.5 1.69) (end 81 1.69) (width 0.5) (layer B.Cu) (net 26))
 (segment (start 61.5 1.69) (end 71.5 1.69) (width 0.5) (layer B.Cu) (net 26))
 (segment (start 51.5 1.69) (end 61.5 1.69) (width 0.5) (layer B.Cu) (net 26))
 (segment (start 41.5 1.69) (end 51.5 1.69) (width 0.5) (layer B.Cu) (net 26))
 (segment (start 31.5 1.69) (end 41.5 1.69) (width 0.5) (layer B.Cu) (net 26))
 (segment (start 21.5 1.69) (end 31.5 1.69) (width 0.5) (layer B.Cu) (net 26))
 (segment (start 11.5 1.69) (end 21.5 1.69) (width 0.5) (layer B.Cu) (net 26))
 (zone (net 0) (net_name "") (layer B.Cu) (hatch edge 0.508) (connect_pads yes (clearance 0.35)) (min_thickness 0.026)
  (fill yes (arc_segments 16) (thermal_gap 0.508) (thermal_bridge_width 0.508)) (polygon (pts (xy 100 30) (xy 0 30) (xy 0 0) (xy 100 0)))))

